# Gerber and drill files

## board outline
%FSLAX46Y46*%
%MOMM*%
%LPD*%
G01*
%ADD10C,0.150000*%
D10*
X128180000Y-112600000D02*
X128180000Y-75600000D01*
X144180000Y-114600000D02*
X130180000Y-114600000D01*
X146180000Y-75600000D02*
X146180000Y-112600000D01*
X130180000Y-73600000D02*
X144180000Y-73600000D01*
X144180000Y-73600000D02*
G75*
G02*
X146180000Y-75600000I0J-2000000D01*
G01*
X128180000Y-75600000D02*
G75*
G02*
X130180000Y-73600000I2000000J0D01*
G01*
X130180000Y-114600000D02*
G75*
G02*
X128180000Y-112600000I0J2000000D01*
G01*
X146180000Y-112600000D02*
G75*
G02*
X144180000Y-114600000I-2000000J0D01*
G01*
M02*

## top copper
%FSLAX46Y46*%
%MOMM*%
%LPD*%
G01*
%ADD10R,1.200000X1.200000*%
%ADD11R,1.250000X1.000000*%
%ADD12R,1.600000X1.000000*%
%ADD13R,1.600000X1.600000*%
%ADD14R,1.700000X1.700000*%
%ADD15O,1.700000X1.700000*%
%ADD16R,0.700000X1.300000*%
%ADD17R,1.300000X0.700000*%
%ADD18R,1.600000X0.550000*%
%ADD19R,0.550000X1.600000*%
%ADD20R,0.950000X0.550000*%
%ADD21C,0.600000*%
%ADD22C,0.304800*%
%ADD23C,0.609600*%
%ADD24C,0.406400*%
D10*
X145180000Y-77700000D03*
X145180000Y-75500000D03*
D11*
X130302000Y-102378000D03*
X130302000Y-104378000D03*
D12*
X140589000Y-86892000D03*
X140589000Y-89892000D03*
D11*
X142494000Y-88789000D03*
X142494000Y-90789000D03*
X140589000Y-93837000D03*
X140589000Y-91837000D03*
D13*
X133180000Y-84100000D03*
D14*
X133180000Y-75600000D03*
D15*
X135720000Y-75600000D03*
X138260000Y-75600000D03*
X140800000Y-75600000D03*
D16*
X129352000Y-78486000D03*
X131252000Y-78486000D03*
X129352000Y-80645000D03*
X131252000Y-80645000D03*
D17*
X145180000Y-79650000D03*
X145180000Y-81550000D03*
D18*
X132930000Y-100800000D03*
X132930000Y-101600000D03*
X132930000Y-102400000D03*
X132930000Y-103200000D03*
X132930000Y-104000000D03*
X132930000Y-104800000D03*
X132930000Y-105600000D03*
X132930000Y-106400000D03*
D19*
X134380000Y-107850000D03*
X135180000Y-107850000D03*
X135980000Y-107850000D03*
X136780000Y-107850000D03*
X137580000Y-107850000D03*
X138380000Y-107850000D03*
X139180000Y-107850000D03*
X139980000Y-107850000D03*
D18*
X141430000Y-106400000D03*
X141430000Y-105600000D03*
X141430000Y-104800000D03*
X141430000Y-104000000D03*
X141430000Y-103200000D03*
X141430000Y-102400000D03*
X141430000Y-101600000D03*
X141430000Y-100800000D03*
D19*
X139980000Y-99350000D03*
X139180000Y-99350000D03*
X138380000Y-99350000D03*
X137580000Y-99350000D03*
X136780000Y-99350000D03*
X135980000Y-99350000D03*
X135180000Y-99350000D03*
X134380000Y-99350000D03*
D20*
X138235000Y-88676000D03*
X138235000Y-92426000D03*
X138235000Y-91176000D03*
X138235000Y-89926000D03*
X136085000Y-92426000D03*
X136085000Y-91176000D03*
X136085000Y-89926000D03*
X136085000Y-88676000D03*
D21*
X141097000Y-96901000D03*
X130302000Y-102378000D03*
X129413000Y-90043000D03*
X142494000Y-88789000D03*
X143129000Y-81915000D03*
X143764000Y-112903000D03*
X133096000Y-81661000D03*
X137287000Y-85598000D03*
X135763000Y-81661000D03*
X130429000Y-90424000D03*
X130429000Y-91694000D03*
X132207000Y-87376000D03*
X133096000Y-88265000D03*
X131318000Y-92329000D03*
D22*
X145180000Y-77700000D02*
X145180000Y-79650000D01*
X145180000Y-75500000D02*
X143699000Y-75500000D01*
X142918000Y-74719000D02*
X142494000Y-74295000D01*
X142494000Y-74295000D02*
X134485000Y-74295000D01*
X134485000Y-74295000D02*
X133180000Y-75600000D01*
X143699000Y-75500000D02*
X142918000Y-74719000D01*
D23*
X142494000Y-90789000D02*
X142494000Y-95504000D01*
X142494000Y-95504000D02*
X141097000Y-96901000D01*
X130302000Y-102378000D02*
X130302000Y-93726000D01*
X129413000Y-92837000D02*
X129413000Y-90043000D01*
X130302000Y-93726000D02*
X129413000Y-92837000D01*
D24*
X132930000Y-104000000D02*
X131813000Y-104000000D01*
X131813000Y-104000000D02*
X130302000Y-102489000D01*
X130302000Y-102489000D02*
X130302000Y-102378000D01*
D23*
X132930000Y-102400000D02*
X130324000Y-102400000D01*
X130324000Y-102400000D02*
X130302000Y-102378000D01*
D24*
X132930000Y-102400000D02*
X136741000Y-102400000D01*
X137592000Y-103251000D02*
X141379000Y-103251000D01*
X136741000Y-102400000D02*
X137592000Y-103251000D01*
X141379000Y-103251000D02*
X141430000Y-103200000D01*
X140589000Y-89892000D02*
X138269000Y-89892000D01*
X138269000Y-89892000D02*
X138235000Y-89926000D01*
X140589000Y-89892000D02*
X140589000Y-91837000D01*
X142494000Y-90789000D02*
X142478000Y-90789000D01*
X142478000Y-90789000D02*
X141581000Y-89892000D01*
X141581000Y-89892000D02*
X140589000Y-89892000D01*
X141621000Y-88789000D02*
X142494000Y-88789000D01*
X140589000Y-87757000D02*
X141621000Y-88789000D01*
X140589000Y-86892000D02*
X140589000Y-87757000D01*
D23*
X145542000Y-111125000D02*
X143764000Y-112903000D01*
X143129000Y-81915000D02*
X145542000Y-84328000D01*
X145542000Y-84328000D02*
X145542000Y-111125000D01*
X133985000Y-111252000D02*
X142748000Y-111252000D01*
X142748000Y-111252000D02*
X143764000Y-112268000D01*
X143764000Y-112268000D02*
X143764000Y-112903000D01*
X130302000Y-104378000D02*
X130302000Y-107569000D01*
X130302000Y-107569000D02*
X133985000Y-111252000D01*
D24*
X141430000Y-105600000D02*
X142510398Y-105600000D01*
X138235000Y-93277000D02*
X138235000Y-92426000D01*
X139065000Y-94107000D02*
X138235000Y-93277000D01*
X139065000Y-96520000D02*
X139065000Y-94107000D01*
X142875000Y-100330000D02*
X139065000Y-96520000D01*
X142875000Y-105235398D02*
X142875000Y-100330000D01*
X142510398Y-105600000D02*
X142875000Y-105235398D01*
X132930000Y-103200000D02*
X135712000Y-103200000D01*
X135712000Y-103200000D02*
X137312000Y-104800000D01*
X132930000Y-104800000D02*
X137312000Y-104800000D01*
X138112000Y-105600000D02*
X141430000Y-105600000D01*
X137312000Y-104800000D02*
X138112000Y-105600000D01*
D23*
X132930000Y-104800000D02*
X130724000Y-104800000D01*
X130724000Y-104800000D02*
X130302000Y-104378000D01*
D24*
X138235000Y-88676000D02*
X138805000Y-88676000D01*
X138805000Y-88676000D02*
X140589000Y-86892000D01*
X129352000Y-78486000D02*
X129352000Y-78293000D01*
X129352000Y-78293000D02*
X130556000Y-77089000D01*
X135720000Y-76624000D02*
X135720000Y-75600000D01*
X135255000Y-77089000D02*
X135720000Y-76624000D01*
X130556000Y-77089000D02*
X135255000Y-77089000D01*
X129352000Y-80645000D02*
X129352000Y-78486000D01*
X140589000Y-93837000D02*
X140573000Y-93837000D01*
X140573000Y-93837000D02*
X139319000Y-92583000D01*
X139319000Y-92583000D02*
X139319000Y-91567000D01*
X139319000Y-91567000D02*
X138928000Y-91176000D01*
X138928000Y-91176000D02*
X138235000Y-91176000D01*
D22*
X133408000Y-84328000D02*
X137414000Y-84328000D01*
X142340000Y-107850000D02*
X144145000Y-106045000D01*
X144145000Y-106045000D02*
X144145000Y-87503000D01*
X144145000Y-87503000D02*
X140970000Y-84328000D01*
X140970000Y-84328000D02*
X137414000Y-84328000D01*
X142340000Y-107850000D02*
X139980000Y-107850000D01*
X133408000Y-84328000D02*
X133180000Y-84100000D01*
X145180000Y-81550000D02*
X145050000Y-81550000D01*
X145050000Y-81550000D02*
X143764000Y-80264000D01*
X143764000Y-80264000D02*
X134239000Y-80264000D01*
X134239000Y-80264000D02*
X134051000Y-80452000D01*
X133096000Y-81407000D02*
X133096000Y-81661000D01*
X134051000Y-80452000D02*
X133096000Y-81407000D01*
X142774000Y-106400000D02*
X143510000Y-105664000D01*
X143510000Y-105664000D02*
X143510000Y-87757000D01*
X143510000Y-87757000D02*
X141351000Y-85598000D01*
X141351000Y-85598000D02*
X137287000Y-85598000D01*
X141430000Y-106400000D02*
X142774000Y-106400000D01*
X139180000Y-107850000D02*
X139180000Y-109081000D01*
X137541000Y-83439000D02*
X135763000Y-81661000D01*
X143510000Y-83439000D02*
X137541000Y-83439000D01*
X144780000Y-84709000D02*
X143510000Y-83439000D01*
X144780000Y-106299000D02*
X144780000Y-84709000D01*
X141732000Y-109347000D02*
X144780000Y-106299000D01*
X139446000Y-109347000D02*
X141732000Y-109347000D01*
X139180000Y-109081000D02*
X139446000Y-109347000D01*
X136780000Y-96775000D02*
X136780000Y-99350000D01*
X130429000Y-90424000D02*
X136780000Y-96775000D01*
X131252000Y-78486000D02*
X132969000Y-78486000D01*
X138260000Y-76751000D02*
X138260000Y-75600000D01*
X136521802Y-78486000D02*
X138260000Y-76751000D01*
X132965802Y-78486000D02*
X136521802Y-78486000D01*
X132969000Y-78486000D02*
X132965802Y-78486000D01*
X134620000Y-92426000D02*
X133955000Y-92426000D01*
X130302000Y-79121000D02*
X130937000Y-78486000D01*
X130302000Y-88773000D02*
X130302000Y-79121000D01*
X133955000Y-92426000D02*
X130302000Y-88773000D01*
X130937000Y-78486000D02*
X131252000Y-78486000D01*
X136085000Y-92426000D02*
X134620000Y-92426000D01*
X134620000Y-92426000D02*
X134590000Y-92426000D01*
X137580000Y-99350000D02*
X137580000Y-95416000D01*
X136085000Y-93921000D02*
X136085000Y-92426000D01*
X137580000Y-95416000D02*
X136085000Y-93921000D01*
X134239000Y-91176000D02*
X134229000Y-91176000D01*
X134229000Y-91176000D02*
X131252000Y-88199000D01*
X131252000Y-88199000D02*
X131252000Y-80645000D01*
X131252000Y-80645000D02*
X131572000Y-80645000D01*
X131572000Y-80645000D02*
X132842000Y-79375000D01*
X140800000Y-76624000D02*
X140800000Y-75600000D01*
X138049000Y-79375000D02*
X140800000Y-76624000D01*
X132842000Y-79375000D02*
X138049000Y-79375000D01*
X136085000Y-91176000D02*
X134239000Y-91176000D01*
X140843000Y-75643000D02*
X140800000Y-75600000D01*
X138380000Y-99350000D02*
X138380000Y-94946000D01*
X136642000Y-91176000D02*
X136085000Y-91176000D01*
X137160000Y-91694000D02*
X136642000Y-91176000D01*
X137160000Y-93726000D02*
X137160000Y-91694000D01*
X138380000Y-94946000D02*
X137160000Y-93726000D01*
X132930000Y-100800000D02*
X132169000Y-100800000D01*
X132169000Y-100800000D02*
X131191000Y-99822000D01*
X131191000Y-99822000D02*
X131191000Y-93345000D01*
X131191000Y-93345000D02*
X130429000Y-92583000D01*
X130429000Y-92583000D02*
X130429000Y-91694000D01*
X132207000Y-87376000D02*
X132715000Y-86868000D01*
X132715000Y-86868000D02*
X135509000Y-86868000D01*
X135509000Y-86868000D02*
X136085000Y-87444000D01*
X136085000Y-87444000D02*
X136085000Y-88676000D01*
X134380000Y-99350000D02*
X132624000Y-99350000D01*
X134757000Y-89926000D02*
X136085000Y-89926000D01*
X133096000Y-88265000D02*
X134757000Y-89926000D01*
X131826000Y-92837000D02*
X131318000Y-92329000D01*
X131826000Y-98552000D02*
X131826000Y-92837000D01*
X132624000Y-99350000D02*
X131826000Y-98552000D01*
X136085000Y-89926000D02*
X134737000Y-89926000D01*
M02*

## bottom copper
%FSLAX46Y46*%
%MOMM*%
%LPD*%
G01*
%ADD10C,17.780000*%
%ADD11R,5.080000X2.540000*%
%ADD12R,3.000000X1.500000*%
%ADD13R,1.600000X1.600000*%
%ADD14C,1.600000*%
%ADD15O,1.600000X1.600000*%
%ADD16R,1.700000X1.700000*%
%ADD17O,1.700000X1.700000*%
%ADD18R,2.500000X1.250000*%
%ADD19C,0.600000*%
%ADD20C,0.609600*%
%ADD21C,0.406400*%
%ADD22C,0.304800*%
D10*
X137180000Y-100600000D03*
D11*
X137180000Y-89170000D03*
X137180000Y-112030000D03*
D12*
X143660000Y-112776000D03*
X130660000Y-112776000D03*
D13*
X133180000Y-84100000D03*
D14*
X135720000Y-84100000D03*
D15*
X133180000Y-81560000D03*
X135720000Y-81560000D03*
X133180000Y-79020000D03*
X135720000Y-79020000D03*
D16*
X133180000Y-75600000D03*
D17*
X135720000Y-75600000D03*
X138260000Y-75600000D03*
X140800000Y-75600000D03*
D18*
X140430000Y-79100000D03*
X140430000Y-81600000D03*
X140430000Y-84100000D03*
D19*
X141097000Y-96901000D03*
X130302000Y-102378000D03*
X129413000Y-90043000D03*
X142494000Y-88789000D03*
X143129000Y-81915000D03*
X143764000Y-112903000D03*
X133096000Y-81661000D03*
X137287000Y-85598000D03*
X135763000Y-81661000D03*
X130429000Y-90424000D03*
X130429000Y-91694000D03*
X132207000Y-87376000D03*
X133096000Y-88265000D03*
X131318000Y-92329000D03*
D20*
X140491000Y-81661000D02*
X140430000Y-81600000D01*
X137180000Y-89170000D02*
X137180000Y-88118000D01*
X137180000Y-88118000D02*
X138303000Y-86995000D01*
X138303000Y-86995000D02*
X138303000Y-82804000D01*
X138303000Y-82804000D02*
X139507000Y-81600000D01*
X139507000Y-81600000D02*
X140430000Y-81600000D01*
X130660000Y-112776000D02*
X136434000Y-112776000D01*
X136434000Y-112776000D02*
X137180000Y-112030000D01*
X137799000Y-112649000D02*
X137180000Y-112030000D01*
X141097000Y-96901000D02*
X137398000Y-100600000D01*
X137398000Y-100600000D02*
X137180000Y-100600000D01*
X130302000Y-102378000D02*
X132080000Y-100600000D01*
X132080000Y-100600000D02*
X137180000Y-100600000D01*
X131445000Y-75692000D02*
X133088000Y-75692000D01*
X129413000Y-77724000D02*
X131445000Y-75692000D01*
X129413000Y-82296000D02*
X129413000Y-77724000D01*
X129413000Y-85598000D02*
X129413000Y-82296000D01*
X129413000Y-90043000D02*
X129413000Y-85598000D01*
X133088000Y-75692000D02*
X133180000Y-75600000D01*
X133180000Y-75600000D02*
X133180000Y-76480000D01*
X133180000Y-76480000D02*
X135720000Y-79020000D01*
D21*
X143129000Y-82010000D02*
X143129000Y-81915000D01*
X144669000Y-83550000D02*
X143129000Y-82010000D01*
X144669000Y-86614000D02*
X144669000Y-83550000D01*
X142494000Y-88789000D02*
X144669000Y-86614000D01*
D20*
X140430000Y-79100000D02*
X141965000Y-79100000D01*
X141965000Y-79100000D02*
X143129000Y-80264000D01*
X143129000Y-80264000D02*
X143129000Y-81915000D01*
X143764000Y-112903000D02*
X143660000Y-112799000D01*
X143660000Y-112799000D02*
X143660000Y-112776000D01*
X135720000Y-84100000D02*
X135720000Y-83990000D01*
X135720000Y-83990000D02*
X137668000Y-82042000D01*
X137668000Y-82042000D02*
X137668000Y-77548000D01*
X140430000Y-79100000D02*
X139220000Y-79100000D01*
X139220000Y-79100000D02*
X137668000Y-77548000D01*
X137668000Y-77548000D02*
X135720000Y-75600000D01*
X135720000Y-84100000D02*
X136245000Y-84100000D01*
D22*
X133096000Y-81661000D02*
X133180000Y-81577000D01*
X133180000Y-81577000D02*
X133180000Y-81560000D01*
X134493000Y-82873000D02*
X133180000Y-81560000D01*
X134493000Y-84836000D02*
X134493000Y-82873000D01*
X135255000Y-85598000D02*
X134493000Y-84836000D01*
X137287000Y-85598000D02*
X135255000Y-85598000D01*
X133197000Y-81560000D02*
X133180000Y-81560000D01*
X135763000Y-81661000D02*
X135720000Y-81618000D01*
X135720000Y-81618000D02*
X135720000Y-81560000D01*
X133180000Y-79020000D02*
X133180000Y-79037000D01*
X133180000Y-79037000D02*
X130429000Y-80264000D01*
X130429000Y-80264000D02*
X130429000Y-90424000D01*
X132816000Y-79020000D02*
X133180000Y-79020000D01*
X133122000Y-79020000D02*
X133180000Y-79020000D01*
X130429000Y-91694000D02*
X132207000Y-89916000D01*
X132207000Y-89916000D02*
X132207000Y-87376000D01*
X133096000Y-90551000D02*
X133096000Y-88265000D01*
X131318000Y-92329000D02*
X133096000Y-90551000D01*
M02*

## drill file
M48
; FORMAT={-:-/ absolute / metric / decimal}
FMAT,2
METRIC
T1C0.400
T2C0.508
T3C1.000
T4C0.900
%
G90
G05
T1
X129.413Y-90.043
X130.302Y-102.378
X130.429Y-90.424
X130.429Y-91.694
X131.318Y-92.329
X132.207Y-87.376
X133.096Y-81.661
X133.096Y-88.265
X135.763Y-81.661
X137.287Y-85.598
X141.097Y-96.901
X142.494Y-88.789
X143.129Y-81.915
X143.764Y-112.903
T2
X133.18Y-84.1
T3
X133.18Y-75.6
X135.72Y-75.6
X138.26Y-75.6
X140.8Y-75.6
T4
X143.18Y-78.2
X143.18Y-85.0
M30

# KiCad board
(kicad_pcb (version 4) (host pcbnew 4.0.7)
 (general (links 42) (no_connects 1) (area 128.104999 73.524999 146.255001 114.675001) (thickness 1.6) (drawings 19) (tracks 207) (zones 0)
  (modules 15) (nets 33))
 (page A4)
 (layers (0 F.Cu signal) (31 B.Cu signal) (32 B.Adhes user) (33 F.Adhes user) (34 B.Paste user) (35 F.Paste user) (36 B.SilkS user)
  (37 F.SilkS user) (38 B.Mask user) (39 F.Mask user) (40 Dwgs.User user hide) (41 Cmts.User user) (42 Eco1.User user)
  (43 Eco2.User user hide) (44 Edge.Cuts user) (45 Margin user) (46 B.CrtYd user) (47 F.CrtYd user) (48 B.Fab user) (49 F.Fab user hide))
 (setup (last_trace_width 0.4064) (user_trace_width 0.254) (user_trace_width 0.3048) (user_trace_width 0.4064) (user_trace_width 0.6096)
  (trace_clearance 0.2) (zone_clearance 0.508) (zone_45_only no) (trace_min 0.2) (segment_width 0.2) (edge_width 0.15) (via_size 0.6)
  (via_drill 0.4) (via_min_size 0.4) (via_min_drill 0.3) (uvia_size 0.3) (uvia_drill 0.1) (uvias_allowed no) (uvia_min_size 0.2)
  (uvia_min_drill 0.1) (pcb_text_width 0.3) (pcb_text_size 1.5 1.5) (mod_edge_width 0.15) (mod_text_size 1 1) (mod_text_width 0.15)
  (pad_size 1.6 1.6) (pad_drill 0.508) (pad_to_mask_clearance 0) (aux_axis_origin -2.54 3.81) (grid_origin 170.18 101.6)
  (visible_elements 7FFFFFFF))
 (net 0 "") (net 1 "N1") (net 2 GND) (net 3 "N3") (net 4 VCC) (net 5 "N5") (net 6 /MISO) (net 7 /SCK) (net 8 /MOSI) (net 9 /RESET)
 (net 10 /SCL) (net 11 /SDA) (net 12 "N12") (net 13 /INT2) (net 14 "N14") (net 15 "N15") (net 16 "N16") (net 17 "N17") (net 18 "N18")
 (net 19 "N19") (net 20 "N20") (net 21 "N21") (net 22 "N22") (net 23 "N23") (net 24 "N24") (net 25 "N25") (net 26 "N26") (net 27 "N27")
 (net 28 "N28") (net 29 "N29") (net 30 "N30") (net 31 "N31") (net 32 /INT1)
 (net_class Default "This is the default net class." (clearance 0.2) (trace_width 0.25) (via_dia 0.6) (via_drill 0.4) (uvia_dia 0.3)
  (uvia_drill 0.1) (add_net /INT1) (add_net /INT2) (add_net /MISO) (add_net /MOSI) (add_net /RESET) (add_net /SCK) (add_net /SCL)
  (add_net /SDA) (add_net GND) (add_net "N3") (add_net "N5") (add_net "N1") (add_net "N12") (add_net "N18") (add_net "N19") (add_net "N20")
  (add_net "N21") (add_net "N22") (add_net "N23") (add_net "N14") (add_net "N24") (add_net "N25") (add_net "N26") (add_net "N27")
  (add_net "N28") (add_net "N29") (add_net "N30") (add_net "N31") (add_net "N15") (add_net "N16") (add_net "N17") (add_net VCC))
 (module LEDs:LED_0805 (layer F.Cu) (at 145.18 76.6 270)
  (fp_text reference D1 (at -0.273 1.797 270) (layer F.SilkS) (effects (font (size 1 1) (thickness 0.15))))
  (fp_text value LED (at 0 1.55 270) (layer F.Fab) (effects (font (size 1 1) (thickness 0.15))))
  (pad 2 smd rect (at 1.1 0 90) (size 1.2 1.2) (layers F.Cu F.Paste F.Mask) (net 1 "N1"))
  (pad 1 smd rect (at -1.1 0 90) (size 1.2 1.2) (layers F.Cu F.Paste F.Mask) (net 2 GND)))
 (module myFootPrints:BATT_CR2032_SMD (layer B.Cu) (at 137.18 100.6 270)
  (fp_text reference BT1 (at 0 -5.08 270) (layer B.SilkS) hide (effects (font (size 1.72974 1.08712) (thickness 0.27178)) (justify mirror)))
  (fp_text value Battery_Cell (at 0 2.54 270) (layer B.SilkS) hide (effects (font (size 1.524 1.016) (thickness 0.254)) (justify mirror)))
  (pad 2 smd circle (at 0 0 270) (size 17.78 17.78) (layers B.Cu B.Paste B.Mask) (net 2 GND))
  (pad 1 smd rect (at -11.43 0 270) (size 2.54 5.08) (layers B.Cu B.Paste B.Mask) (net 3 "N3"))
  (pad 1 smd rect (at 11.43 0 270) (size 2.54 5.08) (layers B.Cu B.Paste B.Mask) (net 3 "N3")))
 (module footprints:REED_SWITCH (layer B.Cu) (at 137.16 112.776 180)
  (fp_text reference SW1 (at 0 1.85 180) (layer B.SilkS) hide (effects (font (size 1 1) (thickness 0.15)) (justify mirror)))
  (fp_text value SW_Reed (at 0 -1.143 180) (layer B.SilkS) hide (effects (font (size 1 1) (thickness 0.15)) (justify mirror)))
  (pad 1 smd rect (at -6.5 0 180) (size 3 1.5) (layers B.Cu B.Paste B.Mask) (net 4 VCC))
  (pad 2 smd rect (at 6.5 0 180) (size 3 1.5) (layers B.Cu B.Paste B.Mask) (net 3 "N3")))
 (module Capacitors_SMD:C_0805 (layer F.Cu) (at 130.302 103.378 270)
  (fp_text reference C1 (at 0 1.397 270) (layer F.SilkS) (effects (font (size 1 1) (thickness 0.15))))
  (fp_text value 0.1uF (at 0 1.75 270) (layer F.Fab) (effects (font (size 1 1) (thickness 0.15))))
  (pad 1 smd rect (at -1 0 270) (size 1 1.25) (layers F.Cu F.Paste F.Mask) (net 2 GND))
  (pad 2 smd rect (at 1 0 270) (size 1 1.25) (layers F.Cu F.Paste F.Mask) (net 4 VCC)))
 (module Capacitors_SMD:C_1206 (layer F.Cu) (at 140.589 88.392 270)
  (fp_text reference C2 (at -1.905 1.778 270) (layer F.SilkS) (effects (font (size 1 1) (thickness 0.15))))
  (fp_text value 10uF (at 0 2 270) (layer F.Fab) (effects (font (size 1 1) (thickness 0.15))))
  (pad 1 smd rect (at -1.5 0 270) (size 1 1.6) (layers F.Cu F.Paste F.Mask) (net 4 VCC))
  (pad 2 smd rect (at 1.5 0 270) (size 1 1.6) (layers F.Cu F.Paste F.Mask) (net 2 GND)))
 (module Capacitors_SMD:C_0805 (layer F.Cu) (at 142.494 89.789 270)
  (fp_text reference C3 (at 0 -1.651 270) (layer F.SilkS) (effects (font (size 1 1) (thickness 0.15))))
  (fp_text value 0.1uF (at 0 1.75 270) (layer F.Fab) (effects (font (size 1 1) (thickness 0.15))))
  (pad 1 smd rect (at -1 0 270) (size 1 1.25) (layers F.Cu F.Paste F.Mask) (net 4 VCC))
  (pad 2 smd rect (at 1 0 270) (size 1 1.25) (layers F.Cu F.Paste F.Mask) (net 2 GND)))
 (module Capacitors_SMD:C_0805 (layer F.Cu) (at 140.589 92.837 90)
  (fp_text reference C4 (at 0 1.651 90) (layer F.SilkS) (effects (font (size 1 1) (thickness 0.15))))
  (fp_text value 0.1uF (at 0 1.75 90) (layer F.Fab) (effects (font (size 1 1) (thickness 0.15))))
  (pad 1 smd rect (at -1 0 90) (size 1 1.25) (layers F.Cu F.Paste F.Mask) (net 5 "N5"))
  (pad 2 smd rect (at 1 0 90) (size 1 1.25) (layers F.Cu F.Paste F.Mask) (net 2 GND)))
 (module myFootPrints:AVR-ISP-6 (layer B.Cu) (at 133.18 84.1)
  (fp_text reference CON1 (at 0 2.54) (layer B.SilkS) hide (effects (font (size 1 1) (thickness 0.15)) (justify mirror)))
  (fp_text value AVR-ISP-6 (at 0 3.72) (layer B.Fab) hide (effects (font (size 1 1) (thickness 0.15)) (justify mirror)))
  (pad 1 thru_hole rect (at 0 0) (size 1.6 1.6) (drill 0.508) (layers *.Cu B.Mask) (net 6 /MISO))
  (pad 2 smd circle (at 2.54 0) (size 1.6 1.6) (layers B.Cu B.Paste B.Mask) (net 4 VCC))
  (pad 3 smd oval (at 0 -2.54) (size 1.6 1.6) (layers B.Cu B.Paste B.Mask) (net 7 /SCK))
  (pad 4 smd oval (at 2.54 -2.54) (size 1.6 1.6) (layers B.Cu B.Paste B.Mask) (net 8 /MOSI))
  (pad 5 smd oval (at 0 -5.08) (size 1.6 1.6) (layers B.Cu B.Paste B.Mask) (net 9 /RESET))
  (pad 6 smd oval (at 2.54 -5.08) (size 1.6 1.6) (layers B.Cu B.Paste B.Mask) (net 2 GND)))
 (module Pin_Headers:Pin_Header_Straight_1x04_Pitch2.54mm (layer F.Cu) (at 133.18 75.6 90)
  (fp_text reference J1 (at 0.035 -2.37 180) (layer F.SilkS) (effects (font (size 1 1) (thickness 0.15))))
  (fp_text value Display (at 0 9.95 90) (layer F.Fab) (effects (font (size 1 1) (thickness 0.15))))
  (pad 1 thru_hole rect (at 0 0 90) (size 1.7 1.7) (drill 1) (layers *.Cu *.Mask) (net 2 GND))
  (pad 2 thru_hole oval (at 0 2.54 90) (size 1.7 1.7) (drill 1) (layers *.Cu *.Mask) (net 4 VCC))
  (pad 3 thru_hole oval (at 0 5.08 90) (size 1.7 1.7) (drill 1) (layers *.Cu *.Mask) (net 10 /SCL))
  (pad 4 thru_hole oval (at 0 7.62 90) (size 1.7 1.7) (drill 1) (layers *.Cu *.Mask) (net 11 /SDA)))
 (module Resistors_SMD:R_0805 (layer F.Cu) (at 130.302 78.486)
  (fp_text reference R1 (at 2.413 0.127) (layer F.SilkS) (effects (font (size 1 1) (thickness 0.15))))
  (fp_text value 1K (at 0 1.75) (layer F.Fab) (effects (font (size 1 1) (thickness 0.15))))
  (pad 1 smd rect (at -0.95 0) (size 0.7 1.3) (layers F.Cu F.Paste F.Mask) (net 4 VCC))
  (pad 2 smd rect (at 0.95 0) (size 0.7 1.3) (layers F.Cu F.Paste F.Mask) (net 10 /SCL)))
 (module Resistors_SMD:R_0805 (layer F.Cu) (at 130.302 80.645)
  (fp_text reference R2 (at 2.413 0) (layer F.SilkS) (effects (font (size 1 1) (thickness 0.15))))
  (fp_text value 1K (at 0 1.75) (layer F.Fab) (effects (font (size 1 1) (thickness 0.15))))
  (pad 1 smd rect (at -0.95 0) (size 0.7 1.3) (layers F.Cu F.Paste F.Mask) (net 4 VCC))
  (pad 2 smd rect (at 0.95 0) (size 0.7 1.3) (layers F.Cu F.Paste F.Mask) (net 11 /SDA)))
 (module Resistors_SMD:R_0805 (layer F.Cu) (at 145.18 80.6 270)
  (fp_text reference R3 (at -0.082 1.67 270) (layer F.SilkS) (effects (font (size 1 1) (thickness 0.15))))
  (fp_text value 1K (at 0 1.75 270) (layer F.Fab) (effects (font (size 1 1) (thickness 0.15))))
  (pad 1 smd rect (at -0.95 0 270) (size 0.7 1.3) (layers F.Cu F.Paste F.Mask) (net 1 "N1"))
  (pad 2 smd rect (at 0.95 0 270) (size 0.7 1.3) (layers F.Cu F.Paste F.Mask) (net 7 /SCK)))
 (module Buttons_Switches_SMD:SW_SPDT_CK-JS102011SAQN (layer B.Cu) (at 143.18 81.6 270)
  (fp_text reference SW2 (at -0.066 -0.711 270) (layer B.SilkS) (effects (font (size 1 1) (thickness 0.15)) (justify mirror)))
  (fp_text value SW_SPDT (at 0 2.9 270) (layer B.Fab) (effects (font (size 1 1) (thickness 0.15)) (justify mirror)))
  (pad 1 smd rect (at -2.5 2.75 270) (size 1.25 2.5) (layers B.Cu B.Paste B.Mask) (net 4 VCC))
  (pad 2 smd rect (at 0 2.75 270) (size 1.25 2.5) (layers B.Cu B.Paste B.Mask) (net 3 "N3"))
  (pad 3 smd rect (at 2.5 2.75 270) (size 1.25 2.5) (layers B.Cu B.Paste B.Mask) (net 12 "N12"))
  (pad "" np_thru_hole circle (at -3.4 0 270) (size 0.9 0.9) (drill 0.9) (layers *.Cu *.Mask))
  (pad "" np_thru_hole circle (at 3.4 0 270) (size 0.9 0.9) (drill 0.9) (layers *.Cu *.Mask)))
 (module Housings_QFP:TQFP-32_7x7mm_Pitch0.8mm (layer F.Cu) (at 137.18 103.6)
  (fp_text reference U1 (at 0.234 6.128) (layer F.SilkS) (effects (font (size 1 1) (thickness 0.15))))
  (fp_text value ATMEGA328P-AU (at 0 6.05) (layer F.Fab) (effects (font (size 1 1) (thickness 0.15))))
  (pad 1 smd rect (at -4.25 -2.8) (size 1.6 0.55) (layers F.Cu F.Paste F.Mask) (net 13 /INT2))
  (pad 2 smd rect (at -4.25 -2) (size 1.6 0.55) (layers F.Cu F.Paste F.Mask) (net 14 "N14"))
  (pad 3 smd rect (at -4.25 -1.2) (size 1.6 0.55) (layers F.Cu F.Paste F.Mask) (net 2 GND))
  (pad 4 smd rect (at -4.25 -0.4) (size 1.6 0.55) (layers F.Cu F.Paste F.Mask) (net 4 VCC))
  (pad 5 smd rect (at -4.25 0.4) (size 1.6 0.55) (layers F.Cu F.Paste F.Mask) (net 2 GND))
  (pad 6 smd rect (at -4.25 1.2) (size 1.6 0.55) (layers F.Cu F.Paste F.Mask) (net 4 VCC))
  (pad 7 smd rect (at -4.25 2) (size 1.6 0.55) (layers F.Cu F.Paste F.Mask) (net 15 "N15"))
  (pad 8 smd rect (at -4.25 2.8) (size 1.6 0.55) (layers F.Cu F.Paste F.Mask) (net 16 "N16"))
  (pad 9 smd rect (at -2.8 4.25 90) (size 1.6 0.55) (layers F.Cu F.Paste F.Mask) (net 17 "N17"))
  (pad 10 smd rect (at -2 4.25 90) (size 1.6 0.55) (layers F.Cu F.Paste F.Mask) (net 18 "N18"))
  (pad 11 smd rect (at -1.2 4.25 90) (size 1.6 0.55) (layers F.Cu F.Paste F.Mask) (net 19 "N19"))
  (pad 12 smd rect (at -0.4 4.25 90) (size 1.6 0.55) (layers F.Cu F.Paste F.Mask) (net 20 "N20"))
  (pad 13 smd rect (at 0.4 4.25 90) (size 1.6 0.55) (layers F.Cu F.Paste F.Mask) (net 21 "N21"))
  (pad 14 smd rect (at 1.2 4.25 90) (size 1.6 0.55) (layers F.Cu F.Paste F.Mask) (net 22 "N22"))
  (pad 15 smd rect (at 2 4.25 90) (size 1.6 0.55) (layers F.Cu F.Paste F.Mask) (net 8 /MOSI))
  (pad 16 smd rect (at 2.8 4.25 90) (size 1.6 0.55) (layers F.Cu F.Paste F.Mask) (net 6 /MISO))
  (pad 17 smd rect (at 4.25 2.8) (size 1.6 0.55) (layers F.Cu F.Paste F.Mask) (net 7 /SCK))
  (pad 18 smd rect (at 4.25 2) (size 1.6 0.55) (layers F.Cu F.Paste F.Mask) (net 4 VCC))
  (pad 19 smd rect (at 4.25 1.2) (size 1.6 0.55) (layers F.Cu F.Paste F.Mask) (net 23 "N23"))
  (pad 20 smd rect (at 4.25 0.4) (size 1.6 0.55) (layers F.Cu F.Paste F.Mask) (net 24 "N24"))
  (pad 21 smd rect (at 4.25 -0.4) (size 1.6 0.55) (layers F.Cu F.Paste F.Mask) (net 2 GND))
  (pad 22 smd rect (at 4.25 -1.2) (size 1.6 0.55) (layers F.Cu F.Paste F.Mask) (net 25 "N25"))
  (pad 23 smd rect (at 4.25 -2) (size 1.6 0.55) (layers F.Cu F.Paste F.Mask) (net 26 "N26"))
  (pad 24 smd rect (at 4.25 -2.8) (size 1.6 0.55) (layers F.Cu F.Paste F.Mask) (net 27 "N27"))
  (pad 25 smd rect (at 2.8 -4.25 90) (size 1.6 0.55) (layers F.Cu F.Paste F.Mask) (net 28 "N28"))
  (pad 26 smd rect (at 2 -4.25 90) (size 1.6 0.55) (layers F.Cu F.Paste F.Mask) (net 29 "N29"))
  (pad 27 smd rect (at 1.2 -4.25 90) (size 1.6 0.55) (layers F.Cu F.Paste F.Mask) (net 11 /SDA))
  (pad 28 smd rect (at 0.4 -4.25 90) (size 1.6 0.55) (layers F.Cu F.Paste F.Mask) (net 10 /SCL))
  (pad 29 smd rect (at -0.4 -4.25 90) (size 1.6 0.55) (layers F.Cu F.Paste F.Mask) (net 9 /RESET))
  (pad 30 smd rect (at -1.2 -4.25 90) (size 1.6 0.55) (layers F.Cu F.Paste F.Mask) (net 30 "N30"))
  (pad 31 smd rect (at -2 -4.25 90) (size 1.6 0.55) (layers F.Cu F.Paste F.Mask) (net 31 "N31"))
  (pad 32 smd rect (at -2.8 -4.25 90) (size 1.6 0.55) (layers F.Cu F.Paste F.Mask) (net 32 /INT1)))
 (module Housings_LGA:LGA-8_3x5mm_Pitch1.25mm (layer F.Cu) (at 137.16 90.551 180)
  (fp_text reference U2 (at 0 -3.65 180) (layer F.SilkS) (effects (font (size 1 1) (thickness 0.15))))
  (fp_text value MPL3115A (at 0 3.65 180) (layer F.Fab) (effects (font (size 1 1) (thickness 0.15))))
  (pad 4 smd rect (at -1.075 1.875 180) (size 0.95 0.55) (layers F.Cu F.Paste F.Mask) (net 4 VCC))
  (pad 1 smd rect (at -1.075 -1.875 180) (size 0.95 0.55) (layers F.Cu F.Paste F.Mask) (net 4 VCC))
  (pad 2 smd rect (at -1.075 -0.625 180) (size 0.95 0.55) (layers F.Cu F.Paste F.Mask) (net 5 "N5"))
  (pad 3 smd rect (at -1.075 0.625 180) (size 0.95 0.55) (layers F.Cu F.Paste F.Mask) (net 2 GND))
  (pad 8 smd rect (at 1.075 -1.875 180) (size 0.95 0.55) (layers F.Cu F.Paste F.Mask) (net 10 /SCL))
  (pad 7 smd rect (at 1.075 -0.625 180) (size 0.95 0.55) (layers F.Cu F.Paste F.Mask) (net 11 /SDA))
  (pad 6 smd rect (at 1.075 0.625 180) (size 0.95 0.55) (layers F.Cu F.Paste F.Mask) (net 32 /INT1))
  (pad 5 smd rect (at 1.075 1.875 180) (size 0.95 0.55) (layers F.Cu F.Paste F.Mask) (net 13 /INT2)))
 (gr_line (start 128.18 112.6) (end 128.18 75.6) (angle 90) (layer Edge.Cuts) (width 0.15))
 (gr_line (start 144.18 114.6) (end 130.18 114.6) (angle 90) (layer Edge.Cuts) (width 0.15))
 (gr_line (start 146.18 75.6) (end 146.18 112.6) (angle 90) (layer Edge.Cuts) (width 0.15))
 (gr_line (start 130.18 73.6) (end 144.18 73.6) (angle 90) (layer Edge.Cuts) (width 0.15))
 (gr_arc (start 144.18 75.6) (end 144.18 73.6) (angle 90) (layer Edge.Cuts) (width 0.15))
 (gr_arc (start 130.18 75.6) (end 128.18 75.6) (angle 90) (layer Edge.Cuts) (width 0.15))
 (gr_arc (start 130.18 112.6) (end 130.18 114.6) (angle 90) (layer Edge.Cuts) (width 0.15))
 (gr_arc (start 144.18 112.6) (end 146.18 112.6) (angle 90) (layer Edge.Cuts) (width 0.15))
 (segment (start 140.491 81.661) (end 140.43 81.6) (width 0.6096) (layer B.Cu) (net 3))
 (segment (start 137.18 89.17) (end 137.18 88.118) (width 0.6096) (layer B.Cu) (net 3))
 (segment (start 137.18 88.118) (end 138.303 86.995) (width 0.6096) (layer B.Cu) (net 3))
 (segment (start 138.303 86.995) (end 138.303 82.804) (width 0.6096) (layer B.Cu) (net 3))
 (segment (start 138.303 82.804) (end 139.507 81.6) (width 0.6096) (layer B.Cu) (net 3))
 (segment (start 139.507 81.6) (end 140.43 81.6) (width 0.6096) (layer B.Cu) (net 3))
 (segment (start 130.66 112.776) (end 136.434 112.776) (width 0.6096) (layer B.Cu) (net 3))
 (segment (start 136.434 112.776) (end 137.18 112.03) (width 0.6096) (layer B.Cu) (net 3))
 (segment (start 137.799 112.649) (end 137.18 112.03) (width 0.6096) (layer B.Cu) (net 3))
 (segment (start 145.18 77.7) (end 145.18 79.65) (width 0.3048) (layer F.Cu) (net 1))
 (segment (start 145.18 75.5) (end 143.699 75.5) (width 0.3048) (layer F.Cu) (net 2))
 (segment (start 142.918 74.719) (end 142.494 74.295) (width 0.3048) (layer F.Cu) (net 2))
 (segment (start 142.494 74.295) (end 134.485 74.295) (width 0.3048) (layer F.Cu) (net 2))
 (segment (start 134.485 74.295) (end 133.18 75.6) (width 0.3048) (layer F.Cu) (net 2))
 (segment (start 143.699 75.5) (end 142.918 74.719) (width 0.3048) (layer F.Cu) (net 2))
 (segment (start 142.494 90.789) (end 142.494 95.504) (width 0.6096) (layer F.Cu) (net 2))
 (segment (start 141.097 96.901) (end 137.398 100.6) (width 0.6096) (layer B.Cu) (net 2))
 (via (at 141.097 96.901) (size 0.6) (drill 0.4) (layers F.Cu B.Cu) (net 2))
 (segment (start 142.494 95.504) (end 141.097 96.901) (width 0.6096) (layer F.Cu) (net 2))
 (segment (start 137.398 100.6) (end 137.18 100.6) (width 0.6096) (layer B.Cu) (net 2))
 (via (at 130.302 102.378) (size 0.6) (drill 0.4) (layers F.Cu B.Cu) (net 2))
 (segment (start 130.302 102.378) (end 132.08 100.6) (width 0.6096) (layer B.Cu) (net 2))
 (segment (start 132.08 100.6) (end 137.18 100.6) (width 0.6096) (layer B.Cu) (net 2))
 (segment (start 130.302 102.378) (end 130.302 93.726) (width 0.6096) (layer F.Cu) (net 2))
 (segment (start 131.445 75.692) (end 133.088 75.692) (width 0.6096) (layer B.Cu) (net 2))
 (segment (start 129.413 77.724) (end 131.445 75.692) (width 0.6096) (layer B.Cu) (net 2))
 (segment (start 129.413 82.296) (end 129.413 77.724) (width 0.6096) (layer B.Cu) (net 2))
 (segment (start 129.413 85.598) (end 129.413 82.296) (width 0.6096) (layer B.Cu) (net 2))
 (segment (start 129.413 90.043) (end 129.413 85.598) (width 0.6096) (layer B.Cu) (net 2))
 (via (at 129.413 90.043) (size 0.6) (drill 0.4) (layers F.Cu B.Cu) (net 2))
 (segment (start 129.413 92.837) (end 129.413 90.043) (width 0.6096) (layer F.Cu) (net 2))
 (segment (start 130.302 93.726) (end 129.413 92.837) (width 0.6096) (layer F.Cu) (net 2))
 (segment (start 133.088 75.692) (end 133.18 75.6) (width 0.6096) (layer B.Cu) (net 2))
 (segment (start 132.93 104) (end 131.813 104) (width 0.4064) (layer F.Cu) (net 2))
 (segment (start 131.813 104) (end 130.302 102.489) (width 0.4064) (layer F.Cu) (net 2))
 (segment (start 130.302 102.489) (end 130.302 102.378) (width 0.4064) (layer F.Cu) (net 2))
 (segment (start 132.93 102.4) (end 130.324 102.4) (width 0.6096) (layer F.Cu) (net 2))
 (segment (start 130.324 102.4) (end 130.302 102.378) (width 0.6096) (layer F.Cu) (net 2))
 (segment (start 132.93 102.4) (end 136.741 102.4) (width 0.4064) (layer F.Cu) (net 2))
 (segment (start 137.592 103.251) (end 141.379 103.251) (width 0.4064) (layer F.Cu) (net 2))
 (segment (start 136.741 102.4) (end 137.592 103.251) (width 0.4064) (layer F.Cu) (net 2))
 (segment (start 141.379 103.251) (end 141.43 103.2) (width 0.4064) (layer F.Cu) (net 2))
 (segment (start 140.589 89.892) (end 138.269 89.892) (width 0.4064) (layer F.Cu) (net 2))
 (segment (start 138.269 89.892) (end 138.235 89.926) (width 0.4064) (layer F.Cu) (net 2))
 (segment (start 140.589 89.892) (end 140.589 91.837) (width 0.4064) (layer F.Cu) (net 2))
 (segment (start 142.494 90.789) (end 142.478 90.789) (width 0.4064) (layer F.Cu) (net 2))
 (segment (start 142.478 90.789) (end 141.581 89.892) (width 0.4064) (layer F.Cu) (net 2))
 (segment (start 141.581 89.892) (end 140.589 89.892) (width 0.4064) (layer F.Cu) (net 2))
 (segment (start 133.18 75.6) (end 133.18 76.48) (width 0.6096) (layer B.Cu) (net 2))
 (segment (start 133.18 76.48) (end 135.72 79.02) (width 0.6096) (layer B.Cu) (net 2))
 (via (at 142.494 88.789) (size 0.6) (drill 0.4) (layers F.Cu B.Cu) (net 4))
 (segment (start 141.621 88.789) (end 142.494 88.789) (width 0.4064) (layer F.Cu) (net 4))
 (segment (start 140.589 87.757) (end 141.621 88.789) (width 0.4064) (layer F.Cu) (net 4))
 (segment (start 140.589 86.892) (end 140.589 87.757) (width 0.4064) (layer F.Cu) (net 4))
 (segment (start 143.129 82.01) (end 143.129 81.915) (width 0.4064) (layer B.Cu) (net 4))
 (segment (start 144.669 83.55) (end 143.129 82.01) (width 0.4064) (layer B.Cu) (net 4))
 (segment (start 144.669 86.614) (end 144.669 83.55) (width 0.4064) (layer B.Cu) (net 4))
 (segment (start 142.494 88.789) (end 144.669 86.614) (width 0.4064) (layer B.Cu) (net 4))
 (segment (start 140.43 79.1) (end 141.965 79.1) (width 0.6096) (layer B.Cu) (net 4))
 (segment (start 141.965 79.1) (end 143.129 80.264) (width 0.6096) (layer B.Cu) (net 4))
 (segment (start 143.129 80.264) (end 143.129 81.915) (width 0.6096) (layer B.Cu) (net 4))
 (segment (start 145.542 111.125) (end 143.764 112.903) (width 0.6096) (layer F.Cu) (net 4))
 (via (at 143.129 81.915) (size 0.6) (drill 0.4) (layers F.Cu B.Cu) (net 4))
 (segment (start 143.129 81.915) (end 145.542 84.328) (width 0.6096) (layer F.Cu) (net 4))
 (segment (start 145.542 84.328) (end 145.542 111.125) (width 0.6096) (layer F.Cu) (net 4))
 (segment (start 133.985 111.252) (end 142.748 111.252) (width 0.6096) (layer F.Cu) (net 4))
 (segment (start 142.748 111.252) (end 143.764 112.268) (width 0.6096) (layer F.Cu) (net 4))
 (segment (start 143.764 112.268) (end 143.764 112.903) (width 0.6096) (layer F.Cu) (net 4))
 (segment (start 130.302 104.378) (end 130.302 107.569) (width 0.6096) (layer F.Cu) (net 4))
 (segment (start 130.302 107.569) (end 133.985 111.252) (width 0.6096) (layer F.Cu) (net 4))
 (segment (start 143.764 112.903) (end 143.66 112.799) (width 0.6096) (layer B.Cu) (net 4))
 (via (at 143.764 112.903) (size 0.6) (drill 0.4) (layers F.Cu B.Cu) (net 4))
 (segment (start 143.66 112.799) (end 143.66 112.776) (width 0.6096) (layer B.Cu) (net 4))
 (segment (start 135.72 84.1) (end 135.72 83.99) (width 0.6096) (layer B.Cu) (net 4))
 (segment (start 135.72 83.99) (end 137.668 82.042) (width 0.6096) (layer B.Cu) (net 4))
 (segment (start 137.668 82.042) (end 137.668 77.548) (width 0.6096) (layer B.Cu) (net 4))
 (segment (start 140.43 79.1) (end 139.22 79.1) (width 0.6096) (layer B.Cu) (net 4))
 (segment (start 139.22 79.1) (end 137.668 77.548) (width 0.6096) (layer B.Cu) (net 4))
 (segment (start 137.668 77.548) (end 135.72 75.6) (width 0.6096) (layer B.Cu) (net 4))
 (segment (start 141.43 105.6) (end 142.510398 105.6) (width 0.4064) (layer F.Cu) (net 4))
 (segment (start 138.235 93.277) (end 138.235 92.426) (width 0.4064) (layer F.Cu) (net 4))
 (segment (start 139.065 94.107) (end 138.235 93.277) (width 0.4064) (layer F.Cu) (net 4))
 (segment (start 139.065 96.52) (end 139.065 94.107) (width 0.4064) (layer F.Cu) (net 4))
 (segment (start 142.875 100.33) (end 139.065 96.52) (width 0.4064) (layer F.Cu) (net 4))
 (segment (start 142.875 105.235398) (end 142.875 100.33) (width 0.4064) (layer F.Cu) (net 4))
 (segment (start 142.510398 105.6) (end 142.875 105.235398) (width 0.4064) (layer F.Cu) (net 4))
 (segment (start 132.93 103.2) (end 135.712 103.2) (width 0.4064) (layer F.Cu) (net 4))
 (segment (start 135.712 103.2) (end 137.312 104.8) (width 0.4064) (layer F.Cu) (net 4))
 (segment (start 132.93 104.8) (end 137.312 104.8) (width 0.4064) (layer F.Cu) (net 4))
 (segment (start 138.112 105.6) (end 141.43 105.6) (width 0.4064) (layer F.Cu) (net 4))
 (segment (start 137.312 104.8) (end 138.112 105.6) (width 0.4064) (layer F.Cu) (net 4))
 (segment (start 132.93 104.8) (end 130.724 104.8) (width 0.6096) (layer F.Cu) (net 4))
 (segment (start 130.724 104.8) (end 130.302 104.378) (width 0.6096) (layer F.Cu) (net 4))
 (segment (start 138.235 88.676) (end 138.805 88.676) (width 0.4064) (layer F.Cu) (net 4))
 (segment (start 138.805 88.676) (end 140.589 86.892) (width 0.4064) (layer F.Cu) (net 4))
 (segment (start 129.352 78.486) (end 129.352 78.293) (width 0.4064) (layer F.Cu) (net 4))
 (segment (start 129.352 78.293) (end 130.556 77.089) (width 0.4064) (layer F.Cu) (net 4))
 (segment (start 135.72 76.624) (end 135.72 75.6) (width 0.4064) (layer F.Cu) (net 4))
 (segment (start 135.255 77.089) (end 135.72 76.624) (width 0.4064) (layer F.Cu) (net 4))
 (segment (start 130.556 77.089) (end 135.255 77.089) (width 0.4064) (layer F.Cu) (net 4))
 (segment (start 129.352 80.645) (end 129.352 78.486) (width 0.4064) (layer F.Cu) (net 4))
 (segment (start 135.72 84.1) (end 136.245 84.1) (width 0.6096) (layer B.Cu) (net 4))
 (segment (start 140.589 93.837) (end 140.573 93.837) (width 0.4064) (layer F.Cu) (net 5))
 (segment (start 140.573 93.837) (end 139.319 92.583) (width 0.4064) (layer F.Cu) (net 5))
 (segment (start 139.319 92.583) (end 139.319 91.567) (width 0.4064) (layer F.Cu) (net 5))
 (segment (start 139.319 91.567) (end 138.928 91.176) (width 0.4064) (layer F.Cu) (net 5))
 (segment (start 138.928 91.176) (end 138.235 91.176) (width 0.4064) (layer F.Cu) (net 5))
 (segment (start 133.408 84.328) (end 137.414 84.328) (width 0.3048) (layer F.Cu) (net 6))
 (segment (start 142.34 107.85) (end 144.145 106.045) (width 0.3048) (layer F.Cu) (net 6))
 (segment (start 144.145 106.045) (end 144.145 87.503) (width 0.3048) (layer F.Cu) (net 6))
 (segment (start 144.145 87.503) (end 140.97 84.328) (width 0.3048) (layer F.Cu) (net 6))
 (segment (start 140.97 84.328) (end 137.414 84.328) (width 0.3048) (layer F.Cu) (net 6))
 (segment (start 142.34 107.85) (end 139.98 107.85) (width 0.3048) (layer F.Cu) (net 6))
 (segment (start 133.408 84.328) (end 133.18 84.1) (width 0.3048) (layer F.Cu) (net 6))
 (segment (start 145.18 81.55) (end 145.05 81.55) (width 0.3048) (layer F.Cu) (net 7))
 (segment (start 145.05 81.55) (end 143.764 80.264) (width 0.3048) (layer F.Cu) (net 7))
 (segment (start 143.764 80.264) (end 134.239 80.264) (width 0.3048) (layer F.Cu) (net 7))
 (segment (start 134.239 80.264) (end 134.051 80.452) (width 0.3048) (layer F.Cu) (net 7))
 (segment (start 133.096 81.661) (end 133.18 81.577) (width 0.3048) (layer B.Cu) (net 7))
 (via (at 133.096 81.661) (size 0.6) (drill 0.4) (layers F.Cu B.Cu) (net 7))
 (segment (start 133.096 81.407) (end 133.096 81.661) (width 0.3048) (layer F.Cu) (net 7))
 (segment (start 134.051 80.452) (end 133.096 81.407) (width 0.3048) (layer F.Cu) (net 7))
 (segment (start 133.18 81.577) (end 133.18 81.56) (width 0.3048) (layer B.Cu) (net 7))
 (via (at 137.287 85.598) (size 0.6) (drill 0.4) (layers F.Cu B.Cu) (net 7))
 (segment (start 142.774 106.4) (end 143.51 105.664) (width 0.3048) (layer F.Cu) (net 7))
 (segment (start 143.51 105.664) (end 143.51 87.757) (width 0.3048) (layer F.Cu) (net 7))
 (segment (start 143.51 87.757) (end 141.351 85.598) (width 0.3048) (layer F.Cu) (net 7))
 (segment (start 141.351 85.598) (end 137.287 85.598) (width 0.3048) (layer F.Cu) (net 7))
 (segment (start 141.43 106.4) (end 142.774 106.4) (width 0.3048) (layer F.Cu) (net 7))
 (segment (start 134.493 82.873) (end 133.18 81.56) (width 0.3048) (layer B.Cu) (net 7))
 (segment (start 134.493 84.836) (end 134.493 82.873) (width 0.3048) (layer B.Cu) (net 7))
 (segment (start 135.255 85.598) (end 134.493 84.836) (width 0.3048) (layer B.Cu) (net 7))
 (segment (start 137.287 85.598) (end 135.255 85.598) (width 0.3048) (layer B.Cu) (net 7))
 (segment (start 133.197 81.56) (end 133.18 81.56) (width 0.3048) (layer B.Cu) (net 7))
 (segment (start 139.18 107.85) (end 139.18 109.081) (width 0.3048) (layer F.Cu) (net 8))
 (segment (start 135.763 81.661) (end 135.72 81.618) (width 0.3048) (layer B.Cu) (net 8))
 (via (at 135.763 81.661) (size 0.6) (drill 0.4) (layers F.Cu B.Cu) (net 8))
 (segment (start 137.541 83.439) (end 135.763 81.661) (width 0.3048) (layer F.Cu) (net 8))
 (segment (start 143.51 83.439) (end 137.541 83.439) (width 0.3048) (layer F.Cu) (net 8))
 (segment (start 144.78 84.709) (end 143.51 83.439) (width 0.3048) (layer F.Cu) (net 8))
 (segment (start 144.78 106.299) (end 144.78 84.709) (width 0.3048) (layer F.Cu) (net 8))
 (segment (start 141.732 109.347) (end 144.78 106.299) (width 0.3048) (layer F.Cu) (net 8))
 (segment (start 139.446 109.347) (end 141.732 109.347) (width 0.3048) (layer F.Cu) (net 8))
 (segment (start 139.18 109.081) (end 139.446 109.347) (width 0.3048) (layer F.Cu) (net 8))
 (segment (start 135.72 81.618) (end 135.72 81.56) (width 0.3048) (layer B.Cu) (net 8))
 (segment (start 133.18 79.02) (end 133.18 79.037) (width 0.3048) (layer B.Cu) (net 9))
 (segment (start 133.18 79.037) (end 130.429 80.264) (width 0.3048) (layer B.Cu) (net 9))
 (segment (start 136.78 96.775) (end 136.78 99.35) (width 0.3048) (layer F.Cu) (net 9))
 (segment (start 130.429 90.424) (end 136.78 96.775) (width 0.3048) (layer F.Cu) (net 9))
 (via (at 130.429 90.424) (size 0.6) (drill 0.4) (layers F.Cu B.Cu) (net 9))
 (segment (start 130.429 80.264) (end 130.429 90.424) (width 0.3048) (layer B.Cu) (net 9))
 (segment (start 132.816 79.02) (end 133.18 79.02) (width 0.3048) (layer B.Cu) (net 9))
 (segment (start 133.122 79.02) (end 133.18 79.02) (width 0.3048) (layer B.Cu) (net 9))
 (segment (start 131.252 78.486) (end 132.969 78.486) (width 0.3048) (layer F.Cu) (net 10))
 (segment (start 138.26 76.751) (end 138.26 75.6) (width 0.3048) (layer F.Cu) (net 10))
 (segment (start 136.521802 78.486) (end 138.26 76.751) (width 0.3048) (layer F.Cu) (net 10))
 (segment (start 132.965802 78.486) (end 136.521802 78.486) (width 0.3048) (layer F.Cu) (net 10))
 (segment (start 132.969 78.486) (end 132.965802 78.486) (width 0.3048) (layer F.Cu) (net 10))
 (segment (start 134.62 92.426) (end 133.955 92.426) (width 0.3048) (layer F.Cu) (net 10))
 (segment (start 130.302 79.121) (end 130.937 78.486) (width 0.3048) (layer F.Cu) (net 10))
 (segment (start 130.302 88.773) (end 130.302 79.121) (width 0.3048) (layer F.Cu) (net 10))
 (segment (start 133.955 92.426) (end 130.302 88.773) (width 0.3048) (layer F.Cu) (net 10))
 (segment (start 130.937 78.486) (end 131.252 78.486) (width 0.3048) (layer F.Cu) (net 10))
 (segment (start 136.085 92.426) (end 134.62 92.426) (width 0.3048) (layer F.Cu) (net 10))
 (segment (start 134.62 92.426) (end 134.59 92.426) (width 0.3048) (layer F.Cu) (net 10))
 (segment (start 137.58 99.35) (end 137.58 95.416) (width 0.3048) (layer F.Cu) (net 10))
 (segment (start 136.085 93.921) (end 136.085 92.426) (width 0.3048) (layer F.Cu) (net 10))
 (segment (start 137.58 95.416) (end 136.085 93.921) (width 0.3048) (layer F.Cu) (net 10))
 (segment (start 134.239 91.176) (end 134.229 91.176) (width 0.3048) (layer F.Cu) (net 11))
 (segment (start 134.229 91.176) (end 131.252 88.199) (width 0.3048) (layer F.Cu) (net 11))
 (segment (start 131.252 88.199) (end 131.252 80.645) (width 0.3048) (layer F.Cu) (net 11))
 (segment (start 131.252 80.645) (end 131.572 80.645) (width 0.3048) (layer F.Cu) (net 11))
 (segment (start 131.572 80.645) (end 132.842 79.375) (width 0.3048) (layer F.Cu) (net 11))
 (segment (start 140.8 76.624) (end 140.8 75.6) (width 0.3048) (layer F.Cu) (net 11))
 (segment (start 138.049 79.375) (end 140.8 76.624) (width 0.3048) (layer F.Cu) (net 11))
 (segment (start 132.842 79.375) (end 138.049 79.375) (width 0.3048) (layer F.Cu) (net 11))
 (segment (start 136.085 91.176) (end 134.239 91.176) (width 0.3048) (layer F.Cu) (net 11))
 (segment (start 140.843 75.643) (end 140.8 75.6) (width 0.3048) (layer F.Cu) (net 11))
 (segment (start 138.38 99.35) (end 138.38 94.946) (width 0.3048) (layer F.Cu) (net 11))
 (segment (start 136.642 91.176) (end 136.085 91.176) (width 0.3048) (layer F.Cu) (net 11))
 (segment (start 137.16 91.694) (end 136.642 91.176) (width 0.3048) (layer F.Cu) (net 11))
 (segment (start 137.16 93.726) (end 137.16 91.694) (width 0.3048) (layer F.Cu) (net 11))
 (segment (start 138.38 94.946) (end 137.16 93.726) (width 0.3048) (layer F.Cu) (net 11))
 (segment (start 132.93 100.8) (end 132.169 100.8) (width 0.3048) (layer F.Cu) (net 13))
 (segment (start 132.169 100.8) (end 131.191 99.822) (width 0.3048) (layer F.Cu) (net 13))
 (segment (start 131.191 99.822) (end 131.191 93.345) (width 0.3048) (layer F.Cu) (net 13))
 (segment (start 131.191 93.345) (end 130.429 92.583) (width 0.3048) (layer F.Cu) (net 13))
 (segment (start 130.429 92.583) (end 130.429 91.694) (width 0.3048) (layer F.Cu) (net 13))
 (via (at 130.429 91.694) (size 0.6) (drill 0.4) (layers F.Cu B.Cu) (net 13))
 (segment (start 130.429 91.694) (end 132.207 89.916) (width 0.3048) (layer B.Cu) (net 13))
 (segment (start 132.207 89.916) (end 132.207 87.376) (width 0.3048) (layer B.Cu) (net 13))
 (via (at 132.207 87.376) (size 0.6) (drill 0.4) (layers F.Cu B.Cu) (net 13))
 (segment (start 132.207 87.376) (end 132.715 86.868) (width 0.3048) (layer F.Cu) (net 13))
 (segment (start 132.715 86.868) (end 135.509 86.868) (width 0.3048) (layer F.Cu) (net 13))
 (segment (start 135.509 86.868) (end 136.085 87.444) (width 0.3048) (layer F.Cu) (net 13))
 (segment (start 136.085 87.444) (end 136.085 88.676) (width 0.3048) (layer F.Cu) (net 13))
 (segment (start 134.38 99.35) (end 132.624 99.35) (width 0.3048) (layer F.Cu) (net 32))
 (segment (start 134.757 89.926) (end 136.085 89.926) (width 0.3048) (layer F.Cu) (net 32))
 (segment (start 133.096 88.265) (end 134.757 89.926) (width 0.3048) (layer F.Cu) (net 32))
 (via (at 133.096 88.265) (size 0.6) (drill 0.4) (layers F.Cu B.Cu) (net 32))
 (segment (start 133.096 90.551) (end 133.096 88.265) (width 0.3048) (layer B.Cu) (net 32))
 (segment (start 131.318 92.329) (end 133.096 90.551) (width 0.3048) (layer B.Cu) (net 32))
 (via (at 131.318 92.329) (size 0.6) (drill 0.4) (layers F.Cu B.Cu) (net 32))
 (segment (start 131.826 92.837) (end 131.318 92.329) (width 0.3048) (layer F.Cu) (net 32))
 (segment (start 131.826 98.552) (end 131.826 92.837) (width 0.3048) (layer F.Cu) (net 32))
 (segment (start 132.624 99.35) (end 131.826 98.552) (width 0.3048) (layer F.Cu) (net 32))
 (segment (start 136.085 89.926) (end 134.737 89.926) (width 0.3048) (layer F.Cu) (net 32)))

